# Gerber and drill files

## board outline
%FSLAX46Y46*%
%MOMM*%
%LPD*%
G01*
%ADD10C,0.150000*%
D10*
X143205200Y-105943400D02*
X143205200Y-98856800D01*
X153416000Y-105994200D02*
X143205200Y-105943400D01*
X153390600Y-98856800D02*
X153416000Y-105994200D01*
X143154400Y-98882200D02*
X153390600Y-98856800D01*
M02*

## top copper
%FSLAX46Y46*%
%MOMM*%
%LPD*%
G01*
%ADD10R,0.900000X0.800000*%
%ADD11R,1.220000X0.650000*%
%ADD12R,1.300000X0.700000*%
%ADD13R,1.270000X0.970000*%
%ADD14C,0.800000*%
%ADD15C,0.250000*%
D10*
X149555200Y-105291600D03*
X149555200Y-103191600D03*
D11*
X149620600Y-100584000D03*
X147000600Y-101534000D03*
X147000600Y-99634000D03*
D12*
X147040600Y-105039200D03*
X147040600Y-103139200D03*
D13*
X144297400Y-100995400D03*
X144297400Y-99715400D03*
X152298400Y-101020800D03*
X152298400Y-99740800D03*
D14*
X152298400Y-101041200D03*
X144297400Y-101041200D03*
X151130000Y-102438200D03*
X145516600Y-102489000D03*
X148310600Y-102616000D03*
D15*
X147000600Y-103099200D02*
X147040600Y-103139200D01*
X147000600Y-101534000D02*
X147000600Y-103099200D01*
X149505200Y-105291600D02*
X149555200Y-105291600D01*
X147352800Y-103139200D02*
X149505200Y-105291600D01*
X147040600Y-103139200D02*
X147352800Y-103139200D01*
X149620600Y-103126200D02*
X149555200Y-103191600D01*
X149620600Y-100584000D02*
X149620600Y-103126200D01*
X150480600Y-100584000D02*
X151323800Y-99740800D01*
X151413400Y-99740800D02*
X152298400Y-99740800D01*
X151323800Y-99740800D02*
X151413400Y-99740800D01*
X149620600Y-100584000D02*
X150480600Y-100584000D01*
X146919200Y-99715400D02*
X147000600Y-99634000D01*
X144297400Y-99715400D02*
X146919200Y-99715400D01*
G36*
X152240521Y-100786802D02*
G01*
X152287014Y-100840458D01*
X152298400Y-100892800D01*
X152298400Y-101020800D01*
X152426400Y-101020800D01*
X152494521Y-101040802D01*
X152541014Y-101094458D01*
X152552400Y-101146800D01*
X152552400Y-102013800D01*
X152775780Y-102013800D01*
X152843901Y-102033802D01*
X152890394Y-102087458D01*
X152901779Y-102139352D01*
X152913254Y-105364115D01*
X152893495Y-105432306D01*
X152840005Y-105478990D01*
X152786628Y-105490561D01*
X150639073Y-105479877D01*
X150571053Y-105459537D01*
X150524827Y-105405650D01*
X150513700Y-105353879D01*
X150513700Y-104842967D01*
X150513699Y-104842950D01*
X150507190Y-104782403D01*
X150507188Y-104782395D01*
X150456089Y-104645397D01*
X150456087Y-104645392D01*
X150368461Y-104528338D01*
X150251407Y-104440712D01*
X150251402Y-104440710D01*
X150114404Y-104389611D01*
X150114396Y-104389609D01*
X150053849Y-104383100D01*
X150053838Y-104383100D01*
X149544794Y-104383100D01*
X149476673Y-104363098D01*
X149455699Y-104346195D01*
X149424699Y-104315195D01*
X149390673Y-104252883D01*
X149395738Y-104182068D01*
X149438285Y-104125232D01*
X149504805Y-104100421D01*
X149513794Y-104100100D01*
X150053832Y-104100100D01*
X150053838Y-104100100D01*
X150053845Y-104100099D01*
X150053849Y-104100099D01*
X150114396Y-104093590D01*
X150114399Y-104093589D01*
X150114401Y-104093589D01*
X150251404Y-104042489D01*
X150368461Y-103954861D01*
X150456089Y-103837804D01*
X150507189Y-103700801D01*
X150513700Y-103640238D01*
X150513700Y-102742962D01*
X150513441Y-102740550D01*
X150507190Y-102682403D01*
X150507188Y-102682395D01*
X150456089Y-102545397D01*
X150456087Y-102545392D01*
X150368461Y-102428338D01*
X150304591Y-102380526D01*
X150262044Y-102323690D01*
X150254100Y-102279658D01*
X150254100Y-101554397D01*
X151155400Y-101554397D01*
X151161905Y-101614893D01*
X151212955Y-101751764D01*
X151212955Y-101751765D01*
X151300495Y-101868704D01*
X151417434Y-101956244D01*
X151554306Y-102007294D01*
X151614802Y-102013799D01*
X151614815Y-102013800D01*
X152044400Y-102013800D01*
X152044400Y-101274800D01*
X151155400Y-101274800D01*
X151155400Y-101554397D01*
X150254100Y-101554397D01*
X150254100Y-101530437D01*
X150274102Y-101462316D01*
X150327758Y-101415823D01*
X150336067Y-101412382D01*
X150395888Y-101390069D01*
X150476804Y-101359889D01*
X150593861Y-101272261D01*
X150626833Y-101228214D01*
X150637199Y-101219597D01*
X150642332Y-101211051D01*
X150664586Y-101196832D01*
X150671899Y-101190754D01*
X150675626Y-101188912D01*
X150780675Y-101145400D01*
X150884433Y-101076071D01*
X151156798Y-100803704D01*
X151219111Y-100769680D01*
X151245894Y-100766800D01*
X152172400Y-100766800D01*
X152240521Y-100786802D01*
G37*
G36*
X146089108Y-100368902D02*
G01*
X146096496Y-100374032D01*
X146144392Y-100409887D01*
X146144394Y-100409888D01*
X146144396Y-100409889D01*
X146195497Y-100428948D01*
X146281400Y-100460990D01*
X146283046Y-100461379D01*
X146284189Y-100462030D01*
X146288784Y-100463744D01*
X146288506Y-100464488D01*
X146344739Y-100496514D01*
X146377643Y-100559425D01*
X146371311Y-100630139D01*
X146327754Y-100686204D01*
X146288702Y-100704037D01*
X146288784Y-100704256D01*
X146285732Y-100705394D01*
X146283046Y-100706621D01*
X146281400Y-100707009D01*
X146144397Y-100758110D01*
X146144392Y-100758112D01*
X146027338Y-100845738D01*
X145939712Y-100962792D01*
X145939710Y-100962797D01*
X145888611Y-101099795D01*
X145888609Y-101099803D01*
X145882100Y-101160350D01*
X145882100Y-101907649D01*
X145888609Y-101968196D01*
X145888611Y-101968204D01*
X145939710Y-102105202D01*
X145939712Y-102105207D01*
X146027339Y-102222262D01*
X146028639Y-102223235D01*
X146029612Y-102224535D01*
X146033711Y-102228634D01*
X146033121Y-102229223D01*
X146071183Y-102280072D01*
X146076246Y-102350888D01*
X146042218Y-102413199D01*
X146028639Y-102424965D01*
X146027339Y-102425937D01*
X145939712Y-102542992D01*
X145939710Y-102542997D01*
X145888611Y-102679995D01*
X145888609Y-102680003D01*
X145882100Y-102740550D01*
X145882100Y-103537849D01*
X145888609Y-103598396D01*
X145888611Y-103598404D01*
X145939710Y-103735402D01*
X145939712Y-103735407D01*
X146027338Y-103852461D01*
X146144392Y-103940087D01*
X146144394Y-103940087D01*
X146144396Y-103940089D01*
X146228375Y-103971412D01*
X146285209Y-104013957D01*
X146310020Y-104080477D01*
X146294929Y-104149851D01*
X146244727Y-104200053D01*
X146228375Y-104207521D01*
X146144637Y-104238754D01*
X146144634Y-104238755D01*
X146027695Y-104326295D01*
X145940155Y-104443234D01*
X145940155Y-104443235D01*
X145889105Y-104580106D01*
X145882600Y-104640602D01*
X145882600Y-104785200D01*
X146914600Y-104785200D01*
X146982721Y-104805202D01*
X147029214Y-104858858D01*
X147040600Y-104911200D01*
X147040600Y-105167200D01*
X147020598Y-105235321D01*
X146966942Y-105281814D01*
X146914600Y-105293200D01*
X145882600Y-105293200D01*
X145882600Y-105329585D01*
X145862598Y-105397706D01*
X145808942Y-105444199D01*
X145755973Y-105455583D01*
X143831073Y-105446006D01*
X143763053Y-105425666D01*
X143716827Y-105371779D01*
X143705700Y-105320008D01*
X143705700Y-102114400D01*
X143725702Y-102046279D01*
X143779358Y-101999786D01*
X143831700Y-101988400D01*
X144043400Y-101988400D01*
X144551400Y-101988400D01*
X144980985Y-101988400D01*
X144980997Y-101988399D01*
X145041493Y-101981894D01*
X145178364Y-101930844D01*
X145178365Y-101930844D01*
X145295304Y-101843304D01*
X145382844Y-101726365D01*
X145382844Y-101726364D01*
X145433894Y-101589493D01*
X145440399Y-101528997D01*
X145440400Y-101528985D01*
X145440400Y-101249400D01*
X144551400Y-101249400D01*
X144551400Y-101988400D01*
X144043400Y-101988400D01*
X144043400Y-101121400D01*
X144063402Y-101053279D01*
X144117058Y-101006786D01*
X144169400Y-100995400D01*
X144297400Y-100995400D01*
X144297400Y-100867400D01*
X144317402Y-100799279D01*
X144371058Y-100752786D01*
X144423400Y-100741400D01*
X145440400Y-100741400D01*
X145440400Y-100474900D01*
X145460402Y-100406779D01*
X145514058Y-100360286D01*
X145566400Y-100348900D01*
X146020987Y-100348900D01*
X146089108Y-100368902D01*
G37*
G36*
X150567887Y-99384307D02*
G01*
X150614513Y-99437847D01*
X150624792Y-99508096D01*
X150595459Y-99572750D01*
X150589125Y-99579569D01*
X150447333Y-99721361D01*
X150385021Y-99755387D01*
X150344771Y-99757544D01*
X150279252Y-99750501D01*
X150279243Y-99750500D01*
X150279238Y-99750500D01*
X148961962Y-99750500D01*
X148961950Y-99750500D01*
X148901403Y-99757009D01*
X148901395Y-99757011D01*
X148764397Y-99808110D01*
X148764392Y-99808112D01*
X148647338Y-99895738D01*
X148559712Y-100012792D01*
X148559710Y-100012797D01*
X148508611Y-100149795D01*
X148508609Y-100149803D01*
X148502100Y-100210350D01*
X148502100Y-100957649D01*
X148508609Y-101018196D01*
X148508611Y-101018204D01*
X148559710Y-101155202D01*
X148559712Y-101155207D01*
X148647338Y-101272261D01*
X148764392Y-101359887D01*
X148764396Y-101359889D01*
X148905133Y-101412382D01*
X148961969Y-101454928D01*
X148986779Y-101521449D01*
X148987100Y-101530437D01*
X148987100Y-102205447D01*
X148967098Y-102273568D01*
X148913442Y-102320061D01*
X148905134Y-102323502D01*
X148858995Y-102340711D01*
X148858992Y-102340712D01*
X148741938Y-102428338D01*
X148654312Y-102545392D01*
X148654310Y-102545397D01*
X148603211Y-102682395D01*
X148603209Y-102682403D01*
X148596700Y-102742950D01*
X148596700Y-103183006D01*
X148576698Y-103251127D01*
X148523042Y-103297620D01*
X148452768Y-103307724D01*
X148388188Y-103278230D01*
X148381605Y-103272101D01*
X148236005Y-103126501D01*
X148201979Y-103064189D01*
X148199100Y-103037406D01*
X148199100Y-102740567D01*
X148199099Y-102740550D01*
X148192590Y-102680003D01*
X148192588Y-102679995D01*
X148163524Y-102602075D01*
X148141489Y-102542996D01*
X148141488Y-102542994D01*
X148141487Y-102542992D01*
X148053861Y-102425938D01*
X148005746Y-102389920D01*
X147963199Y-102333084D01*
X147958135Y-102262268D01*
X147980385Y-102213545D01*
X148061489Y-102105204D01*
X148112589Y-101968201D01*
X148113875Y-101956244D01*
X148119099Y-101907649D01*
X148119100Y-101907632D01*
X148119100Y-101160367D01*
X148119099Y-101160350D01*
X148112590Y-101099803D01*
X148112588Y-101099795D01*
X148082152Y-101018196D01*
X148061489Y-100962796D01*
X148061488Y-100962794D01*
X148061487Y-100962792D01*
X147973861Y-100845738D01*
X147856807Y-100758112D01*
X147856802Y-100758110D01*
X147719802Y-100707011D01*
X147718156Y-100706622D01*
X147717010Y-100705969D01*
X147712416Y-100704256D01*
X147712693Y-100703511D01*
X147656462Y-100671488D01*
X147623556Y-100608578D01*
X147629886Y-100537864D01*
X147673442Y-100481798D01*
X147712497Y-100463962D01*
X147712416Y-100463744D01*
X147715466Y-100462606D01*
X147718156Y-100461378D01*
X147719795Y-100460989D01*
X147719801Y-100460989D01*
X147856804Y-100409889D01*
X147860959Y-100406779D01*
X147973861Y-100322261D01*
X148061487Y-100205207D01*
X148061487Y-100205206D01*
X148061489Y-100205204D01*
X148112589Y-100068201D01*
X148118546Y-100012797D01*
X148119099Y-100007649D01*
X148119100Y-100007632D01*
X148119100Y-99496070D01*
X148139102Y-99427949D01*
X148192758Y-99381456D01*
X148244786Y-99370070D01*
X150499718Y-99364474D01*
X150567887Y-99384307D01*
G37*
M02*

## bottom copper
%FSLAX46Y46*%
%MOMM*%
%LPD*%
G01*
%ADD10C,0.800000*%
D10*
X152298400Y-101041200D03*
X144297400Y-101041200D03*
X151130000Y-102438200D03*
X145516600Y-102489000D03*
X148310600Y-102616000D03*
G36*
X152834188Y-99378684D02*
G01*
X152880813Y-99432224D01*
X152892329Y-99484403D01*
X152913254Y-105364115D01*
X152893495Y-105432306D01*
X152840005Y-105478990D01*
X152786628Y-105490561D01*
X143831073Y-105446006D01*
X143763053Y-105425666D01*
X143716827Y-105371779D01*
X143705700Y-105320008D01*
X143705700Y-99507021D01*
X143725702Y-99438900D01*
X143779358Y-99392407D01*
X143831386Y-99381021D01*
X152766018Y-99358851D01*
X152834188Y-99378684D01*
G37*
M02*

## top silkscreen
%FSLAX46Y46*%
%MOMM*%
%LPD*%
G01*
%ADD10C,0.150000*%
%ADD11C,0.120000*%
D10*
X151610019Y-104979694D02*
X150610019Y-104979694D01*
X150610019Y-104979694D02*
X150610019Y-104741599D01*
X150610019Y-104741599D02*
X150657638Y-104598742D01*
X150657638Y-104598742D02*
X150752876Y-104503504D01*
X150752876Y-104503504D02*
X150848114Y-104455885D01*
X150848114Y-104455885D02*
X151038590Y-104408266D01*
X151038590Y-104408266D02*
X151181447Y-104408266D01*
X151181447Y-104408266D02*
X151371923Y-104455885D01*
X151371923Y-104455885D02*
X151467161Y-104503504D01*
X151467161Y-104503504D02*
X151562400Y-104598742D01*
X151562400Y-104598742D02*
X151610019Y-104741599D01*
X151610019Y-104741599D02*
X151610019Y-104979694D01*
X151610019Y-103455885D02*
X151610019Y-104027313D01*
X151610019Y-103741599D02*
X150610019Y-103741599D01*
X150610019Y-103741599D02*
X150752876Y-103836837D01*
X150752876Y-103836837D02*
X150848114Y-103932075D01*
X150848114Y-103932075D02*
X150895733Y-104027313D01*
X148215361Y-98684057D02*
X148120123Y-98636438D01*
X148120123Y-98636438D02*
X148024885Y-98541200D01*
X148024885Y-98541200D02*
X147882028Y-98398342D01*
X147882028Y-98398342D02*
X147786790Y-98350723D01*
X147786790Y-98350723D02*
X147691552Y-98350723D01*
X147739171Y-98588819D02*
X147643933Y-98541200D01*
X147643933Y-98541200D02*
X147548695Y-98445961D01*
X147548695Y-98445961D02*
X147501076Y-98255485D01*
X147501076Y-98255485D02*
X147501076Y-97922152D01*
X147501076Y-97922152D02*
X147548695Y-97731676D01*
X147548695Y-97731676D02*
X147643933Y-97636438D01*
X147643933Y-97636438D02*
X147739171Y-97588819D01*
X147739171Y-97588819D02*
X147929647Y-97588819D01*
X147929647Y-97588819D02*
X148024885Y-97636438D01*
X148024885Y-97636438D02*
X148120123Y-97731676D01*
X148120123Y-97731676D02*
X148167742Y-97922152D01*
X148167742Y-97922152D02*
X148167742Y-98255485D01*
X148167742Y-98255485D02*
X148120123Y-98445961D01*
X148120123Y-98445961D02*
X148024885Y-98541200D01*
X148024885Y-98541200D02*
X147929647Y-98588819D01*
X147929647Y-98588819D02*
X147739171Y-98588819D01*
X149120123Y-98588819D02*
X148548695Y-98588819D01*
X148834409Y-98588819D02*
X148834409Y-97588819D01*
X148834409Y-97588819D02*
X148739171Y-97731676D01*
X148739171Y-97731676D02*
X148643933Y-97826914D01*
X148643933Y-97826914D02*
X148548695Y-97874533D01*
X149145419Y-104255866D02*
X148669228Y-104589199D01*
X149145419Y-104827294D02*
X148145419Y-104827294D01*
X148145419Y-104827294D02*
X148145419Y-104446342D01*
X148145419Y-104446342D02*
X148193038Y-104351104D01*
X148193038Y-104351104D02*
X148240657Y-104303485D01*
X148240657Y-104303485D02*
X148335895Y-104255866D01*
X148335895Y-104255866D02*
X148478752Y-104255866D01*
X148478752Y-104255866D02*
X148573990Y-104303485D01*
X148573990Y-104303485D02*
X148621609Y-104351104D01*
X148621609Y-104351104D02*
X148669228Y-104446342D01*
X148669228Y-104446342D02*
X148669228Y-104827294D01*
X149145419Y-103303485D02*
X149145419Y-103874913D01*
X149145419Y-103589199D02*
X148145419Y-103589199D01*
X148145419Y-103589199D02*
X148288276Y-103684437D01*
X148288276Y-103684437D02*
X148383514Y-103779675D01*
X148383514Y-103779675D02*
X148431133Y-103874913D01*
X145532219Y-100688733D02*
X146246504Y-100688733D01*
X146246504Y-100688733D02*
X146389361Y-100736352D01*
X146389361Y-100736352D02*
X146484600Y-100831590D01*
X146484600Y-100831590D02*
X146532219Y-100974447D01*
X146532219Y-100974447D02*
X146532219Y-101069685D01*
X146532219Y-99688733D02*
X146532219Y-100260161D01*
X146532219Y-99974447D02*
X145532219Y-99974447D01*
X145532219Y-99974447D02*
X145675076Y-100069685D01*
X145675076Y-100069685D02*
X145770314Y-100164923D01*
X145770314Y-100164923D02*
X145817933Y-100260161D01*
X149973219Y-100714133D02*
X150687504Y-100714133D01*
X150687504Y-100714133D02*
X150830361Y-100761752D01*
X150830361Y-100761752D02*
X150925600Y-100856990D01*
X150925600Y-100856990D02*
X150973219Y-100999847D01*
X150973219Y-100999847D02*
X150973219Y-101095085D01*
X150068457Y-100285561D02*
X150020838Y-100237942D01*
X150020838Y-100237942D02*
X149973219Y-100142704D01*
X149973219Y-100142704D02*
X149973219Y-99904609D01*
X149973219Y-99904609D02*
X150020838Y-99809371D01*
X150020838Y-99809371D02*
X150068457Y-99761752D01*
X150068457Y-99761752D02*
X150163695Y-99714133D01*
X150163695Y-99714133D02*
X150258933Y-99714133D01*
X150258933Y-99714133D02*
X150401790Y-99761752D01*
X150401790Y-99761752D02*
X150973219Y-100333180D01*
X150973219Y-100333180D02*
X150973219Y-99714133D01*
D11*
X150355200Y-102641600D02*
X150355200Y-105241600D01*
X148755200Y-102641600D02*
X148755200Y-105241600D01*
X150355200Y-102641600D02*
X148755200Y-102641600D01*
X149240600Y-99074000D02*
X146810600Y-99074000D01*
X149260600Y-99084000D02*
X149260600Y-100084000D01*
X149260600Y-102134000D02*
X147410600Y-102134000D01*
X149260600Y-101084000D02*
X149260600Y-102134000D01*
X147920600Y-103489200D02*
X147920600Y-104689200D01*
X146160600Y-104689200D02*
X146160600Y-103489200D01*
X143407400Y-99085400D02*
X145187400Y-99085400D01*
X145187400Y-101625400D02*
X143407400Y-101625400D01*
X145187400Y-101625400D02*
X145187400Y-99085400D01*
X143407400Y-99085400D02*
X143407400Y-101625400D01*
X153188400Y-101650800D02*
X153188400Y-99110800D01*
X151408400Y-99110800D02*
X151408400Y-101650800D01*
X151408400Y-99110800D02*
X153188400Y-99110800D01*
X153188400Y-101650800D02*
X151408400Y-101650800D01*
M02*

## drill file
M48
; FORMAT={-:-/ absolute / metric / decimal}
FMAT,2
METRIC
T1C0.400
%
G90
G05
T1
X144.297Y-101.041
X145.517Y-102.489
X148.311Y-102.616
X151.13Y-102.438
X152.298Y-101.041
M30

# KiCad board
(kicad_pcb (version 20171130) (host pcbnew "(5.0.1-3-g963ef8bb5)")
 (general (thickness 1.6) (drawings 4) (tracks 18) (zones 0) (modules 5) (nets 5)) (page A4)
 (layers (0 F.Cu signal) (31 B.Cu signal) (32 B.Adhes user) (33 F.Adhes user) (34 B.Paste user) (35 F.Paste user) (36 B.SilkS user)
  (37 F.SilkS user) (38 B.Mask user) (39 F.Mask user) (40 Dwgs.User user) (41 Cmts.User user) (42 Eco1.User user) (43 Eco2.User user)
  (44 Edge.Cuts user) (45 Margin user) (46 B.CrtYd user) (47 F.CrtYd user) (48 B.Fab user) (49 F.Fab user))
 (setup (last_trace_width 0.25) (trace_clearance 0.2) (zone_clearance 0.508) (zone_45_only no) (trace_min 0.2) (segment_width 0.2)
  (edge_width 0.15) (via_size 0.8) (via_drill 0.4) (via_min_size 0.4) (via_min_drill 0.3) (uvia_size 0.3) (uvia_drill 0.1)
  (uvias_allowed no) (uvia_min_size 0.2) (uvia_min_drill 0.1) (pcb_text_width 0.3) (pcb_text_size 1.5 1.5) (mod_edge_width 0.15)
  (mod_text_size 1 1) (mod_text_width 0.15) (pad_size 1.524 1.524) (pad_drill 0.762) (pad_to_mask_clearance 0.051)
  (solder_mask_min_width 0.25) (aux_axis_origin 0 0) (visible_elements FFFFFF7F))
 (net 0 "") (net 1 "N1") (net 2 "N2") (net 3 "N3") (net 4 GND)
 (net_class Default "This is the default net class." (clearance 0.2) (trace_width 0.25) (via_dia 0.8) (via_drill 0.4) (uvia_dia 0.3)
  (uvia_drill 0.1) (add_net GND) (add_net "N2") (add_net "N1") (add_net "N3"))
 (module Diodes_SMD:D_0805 (layer F.Cu) (at 149.5552 104.2416 270)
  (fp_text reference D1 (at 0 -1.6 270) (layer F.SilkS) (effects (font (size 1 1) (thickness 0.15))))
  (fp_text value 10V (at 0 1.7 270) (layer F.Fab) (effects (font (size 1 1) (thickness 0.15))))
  (fp_line (start -1.6 -0.8) (end 1 -0.8) (layer F.SilkS) (width 0.12))
  (fp_line (start -1.6 0.8) (end 1 0.8) (layer F.SilkS) (width 0.12))
  (fp_line (start -1.6 -0.8) (end -1.6 0.8) (layer F.SilkS) (width 0.12))
  (pad 2 smd rect (at 1.05 0 270) (size 0.8 0.9) (layers F.Cu F.Paste F.Mask) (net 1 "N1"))
  (pad 1 smd rect (at -1.05 0 270) (size 0.8 0.9) (layers F.Cu F.Paste F.Mask) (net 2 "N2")))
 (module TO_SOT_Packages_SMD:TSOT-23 (layer F.Cu) (at 148.3106 100.584)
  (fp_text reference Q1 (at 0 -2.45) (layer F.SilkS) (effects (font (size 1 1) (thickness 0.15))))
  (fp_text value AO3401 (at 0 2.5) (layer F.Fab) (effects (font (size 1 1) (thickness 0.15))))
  (fp_line (start 0.93 -1.51) (end -1.5 -1.51) (layer F.SilkS) (width 0.12))
  (fp_line (start 0.95 -1.5) (end 0.95 -0.5) (layer F.SilkS) (width 0.12))
  (fp_line (start 0.95 1.55) (end -0.9 1.55) (layer F.SilkS) (width 0.12))
  (fp_line (start 0.95 0.5) (end 0.95 1.55) (layer F.SilkS) (width 0.12))
  (pad 3 smd rect (at 1.31 0) (size 1.22 0.65) (layers F.Cu F.Paste F.Mask) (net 2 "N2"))
  (pad 2 smd rect (at -1.31 0.95) (size 1.22 0.65) (layers F.Cu F.Paste F.Mask) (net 1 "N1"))
  (pad 1 smd rect (at -1.31 -0.95) (size 1.22 0.65) (layers F.Cu F.Paste F.Mask) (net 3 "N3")))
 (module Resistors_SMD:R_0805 (layer F.Cu) (at 147.0406 104.0892 270)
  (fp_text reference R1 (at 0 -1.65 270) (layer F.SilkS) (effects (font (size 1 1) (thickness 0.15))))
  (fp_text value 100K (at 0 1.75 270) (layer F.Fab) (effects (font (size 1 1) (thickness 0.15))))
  (fp_line (start -0.6 -0.88) (end 0.6 -0.88) (layer F.SilkS) (width 0.12))
  (fp_line (start 0.6 0.88) (end -0.6 0.88) (layer F.SilkS) (width 0.12))
  (pad 2 smd rect (at 0.95 0 270) (size 0.7 1.3) (layers F.Cu F.Paste F.Mask) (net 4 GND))
  (pad 1 smd rect (at -0.95 0 270) (size 0.7 1.3) (layers F.Cu F.Paste F.Mask) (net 1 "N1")))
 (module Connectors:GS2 (layer F.Cu) (at 144.2974 100.3554)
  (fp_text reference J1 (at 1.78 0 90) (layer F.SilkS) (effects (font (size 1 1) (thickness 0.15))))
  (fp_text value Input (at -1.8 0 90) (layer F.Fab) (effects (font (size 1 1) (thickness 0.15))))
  (fp_line (start -0.89 -1.27) (end 0.89 -1.27) (layer F.SilkS) (width 0.12))
  (fp_line (start 0.89 1.27) (end -0.89 1.27) (layer F.SilkS) (width 0.12))
  (fp_line (start 0.89 1.27) (end 0.89 -1.27) (layer F.SilkS) (width 0.12))
  (fp_line (start -0.89 -1.27) (end -0.89 1.27) (layer F.SilkS) (width 0.12))
  (pad 2 smd rect (at 0 0.64) (size 1.27 0.97) (layers F.Cu F.Paste F.Mask) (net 4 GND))
  (pad 1 smd rect (at 0 -0.64) (size 1.27 0.97) (layers F.Cu F.Paste F.Mask) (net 3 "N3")))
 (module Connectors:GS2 (layer F.Cu) (at 152.2984 100.3808 180)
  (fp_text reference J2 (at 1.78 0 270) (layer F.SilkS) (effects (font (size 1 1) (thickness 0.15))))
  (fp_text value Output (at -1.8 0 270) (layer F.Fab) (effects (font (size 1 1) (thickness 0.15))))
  (fp_line (start -0.89 -1.27) (end -0.89 1.27) (layer F.SilkS) (width 0.12))
  (fp_line (start 0.89 1.27) (end 0.89 -1.27) (layer F.SilkS) (width 0.12))
  (fp_line (start 0.89 1.27) (end -0.89 1.27) (layer F.SilkS) (width 0.12))
  (fp_line (start -0.89 -1.27) (end 0.89 -1.27) (layer F.SilkS) (width 0.12))
  (pad 1 smd rect (at 0 -0.64 180) (size 1.27 0.97) (layers F.Cu F.Paste F.Mask) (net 4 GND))
  (pad 2 smd rect (at 0 0.64 180) (size 1.27 0.97) (layers F.Cu F.Paste F.Mask) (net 2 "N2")))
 (gr_line (start 143.2052 105.9434) (end 143.2052 98.8568) (layer Edge.Cuts) (width 0.15))
 (gr_line (start 153.416 105.9942) (end 143.2052 105.9434) (layer Edge.Cuts) (width 0.15))
 (gr_line (start 153.3906 98.8568) (end 153.416 105.9942) (layer Edge.Cuts) (width 0.15))
 (gr_line (start 143.1544 98.8822) (end 153.3906 98.8568) (layer Edge.Cuts) (width 0.15))
 (via (at 152.2984 101.0412) (size 0.8) (drill 0.4) (layers F.Cu B.Cu) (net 4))
 (via (at 144.2974 101.0412) (size 0.8) (drill 0.4) (layers F.Cu B.Cu) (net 4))
 (segment (start 147.0006 103.0992) (end 147.0406 103.1392) (width 0.25) (layer F.Cu) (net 1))
 (segment (start 147.0006 101.534) (end 147.0006 103.0992) (width 0.25) (layer F.Cu) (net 1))
 (segment (start 149.5052 105.2916) (end 149.5552 105.2916) (width 0.25) (layer F.Cu) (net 1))
 (segment (start 147.3528 103.1392) (end 149.5052 105.2916) (width 0.25) (layer F.Cu) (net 1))
 (segment (start 147.0406 103.1392) (end 147.3528 103.1392) (width 0.25) (layer F.Cu) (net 1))
 (segment (start 149.6206 103.1262) (end 149.5552 103.1916) (width 0.25) (layer F.Cu) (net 2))
 (segment (start 149.6206 100.584) (end 149.6206 103.1262) (width 0.25) (layer F.Cu) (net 2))
 (segment (start 150.4806 100.584) (end 151.3238 99.7408) (width 0.25) (layer F.Cu) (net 2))
 (segment (start 151.4134 99.7408) (end 152.2984 99.7408) (width 0.25) (layer F.Cu) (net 2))
 (segment (start 151.3238 99.7408) (end 151.4134 99.7408) (width 0.25) (layer F.Cu) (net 2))
 (segment (start 149.6206 100.584) (end 150.4806 100.584) (width 0.25) (layer F.Cu) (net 2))
 (segment (start 146.9192 99.7154) (end 147.0006 99.634) (width 0.25) (layer F.Cu) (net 3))
 (segment (start 144.2974 99.7154) (end 146.9192 99.7154) (width 0.25) (layer F.Cu) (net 3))
 (via (at 151.13 102.4382) (size 0.8) (drill 0.4) (layers F.Cu B.Cu) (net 4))
 (via (at 145.5166 102.489) (size 0.8) (drill 0.4) (layers F.Cu B.Cu) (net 4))
 (via (at 148.3106 102.616) (size 0.8) (drill 0.4) (layers F.Cu B.Cu) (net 4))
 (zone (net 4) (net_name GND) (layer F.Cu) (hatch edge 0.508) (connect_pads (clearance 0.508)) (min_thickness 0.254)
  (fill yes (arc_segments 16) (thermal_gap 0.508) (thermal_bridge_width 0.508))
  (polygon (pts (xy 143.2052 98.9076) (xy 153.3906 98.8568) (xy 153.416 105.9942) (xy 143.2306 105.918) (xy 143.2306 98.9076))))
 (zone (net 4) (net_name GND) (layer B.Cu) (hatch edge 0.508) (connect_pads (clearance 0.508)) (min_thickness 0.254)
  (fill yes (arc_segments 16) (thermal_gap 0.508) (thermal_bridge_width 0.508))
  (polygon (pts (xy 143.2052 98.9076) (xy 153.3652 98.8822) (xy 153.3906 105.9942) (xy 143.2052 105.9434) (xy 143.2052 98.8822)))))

